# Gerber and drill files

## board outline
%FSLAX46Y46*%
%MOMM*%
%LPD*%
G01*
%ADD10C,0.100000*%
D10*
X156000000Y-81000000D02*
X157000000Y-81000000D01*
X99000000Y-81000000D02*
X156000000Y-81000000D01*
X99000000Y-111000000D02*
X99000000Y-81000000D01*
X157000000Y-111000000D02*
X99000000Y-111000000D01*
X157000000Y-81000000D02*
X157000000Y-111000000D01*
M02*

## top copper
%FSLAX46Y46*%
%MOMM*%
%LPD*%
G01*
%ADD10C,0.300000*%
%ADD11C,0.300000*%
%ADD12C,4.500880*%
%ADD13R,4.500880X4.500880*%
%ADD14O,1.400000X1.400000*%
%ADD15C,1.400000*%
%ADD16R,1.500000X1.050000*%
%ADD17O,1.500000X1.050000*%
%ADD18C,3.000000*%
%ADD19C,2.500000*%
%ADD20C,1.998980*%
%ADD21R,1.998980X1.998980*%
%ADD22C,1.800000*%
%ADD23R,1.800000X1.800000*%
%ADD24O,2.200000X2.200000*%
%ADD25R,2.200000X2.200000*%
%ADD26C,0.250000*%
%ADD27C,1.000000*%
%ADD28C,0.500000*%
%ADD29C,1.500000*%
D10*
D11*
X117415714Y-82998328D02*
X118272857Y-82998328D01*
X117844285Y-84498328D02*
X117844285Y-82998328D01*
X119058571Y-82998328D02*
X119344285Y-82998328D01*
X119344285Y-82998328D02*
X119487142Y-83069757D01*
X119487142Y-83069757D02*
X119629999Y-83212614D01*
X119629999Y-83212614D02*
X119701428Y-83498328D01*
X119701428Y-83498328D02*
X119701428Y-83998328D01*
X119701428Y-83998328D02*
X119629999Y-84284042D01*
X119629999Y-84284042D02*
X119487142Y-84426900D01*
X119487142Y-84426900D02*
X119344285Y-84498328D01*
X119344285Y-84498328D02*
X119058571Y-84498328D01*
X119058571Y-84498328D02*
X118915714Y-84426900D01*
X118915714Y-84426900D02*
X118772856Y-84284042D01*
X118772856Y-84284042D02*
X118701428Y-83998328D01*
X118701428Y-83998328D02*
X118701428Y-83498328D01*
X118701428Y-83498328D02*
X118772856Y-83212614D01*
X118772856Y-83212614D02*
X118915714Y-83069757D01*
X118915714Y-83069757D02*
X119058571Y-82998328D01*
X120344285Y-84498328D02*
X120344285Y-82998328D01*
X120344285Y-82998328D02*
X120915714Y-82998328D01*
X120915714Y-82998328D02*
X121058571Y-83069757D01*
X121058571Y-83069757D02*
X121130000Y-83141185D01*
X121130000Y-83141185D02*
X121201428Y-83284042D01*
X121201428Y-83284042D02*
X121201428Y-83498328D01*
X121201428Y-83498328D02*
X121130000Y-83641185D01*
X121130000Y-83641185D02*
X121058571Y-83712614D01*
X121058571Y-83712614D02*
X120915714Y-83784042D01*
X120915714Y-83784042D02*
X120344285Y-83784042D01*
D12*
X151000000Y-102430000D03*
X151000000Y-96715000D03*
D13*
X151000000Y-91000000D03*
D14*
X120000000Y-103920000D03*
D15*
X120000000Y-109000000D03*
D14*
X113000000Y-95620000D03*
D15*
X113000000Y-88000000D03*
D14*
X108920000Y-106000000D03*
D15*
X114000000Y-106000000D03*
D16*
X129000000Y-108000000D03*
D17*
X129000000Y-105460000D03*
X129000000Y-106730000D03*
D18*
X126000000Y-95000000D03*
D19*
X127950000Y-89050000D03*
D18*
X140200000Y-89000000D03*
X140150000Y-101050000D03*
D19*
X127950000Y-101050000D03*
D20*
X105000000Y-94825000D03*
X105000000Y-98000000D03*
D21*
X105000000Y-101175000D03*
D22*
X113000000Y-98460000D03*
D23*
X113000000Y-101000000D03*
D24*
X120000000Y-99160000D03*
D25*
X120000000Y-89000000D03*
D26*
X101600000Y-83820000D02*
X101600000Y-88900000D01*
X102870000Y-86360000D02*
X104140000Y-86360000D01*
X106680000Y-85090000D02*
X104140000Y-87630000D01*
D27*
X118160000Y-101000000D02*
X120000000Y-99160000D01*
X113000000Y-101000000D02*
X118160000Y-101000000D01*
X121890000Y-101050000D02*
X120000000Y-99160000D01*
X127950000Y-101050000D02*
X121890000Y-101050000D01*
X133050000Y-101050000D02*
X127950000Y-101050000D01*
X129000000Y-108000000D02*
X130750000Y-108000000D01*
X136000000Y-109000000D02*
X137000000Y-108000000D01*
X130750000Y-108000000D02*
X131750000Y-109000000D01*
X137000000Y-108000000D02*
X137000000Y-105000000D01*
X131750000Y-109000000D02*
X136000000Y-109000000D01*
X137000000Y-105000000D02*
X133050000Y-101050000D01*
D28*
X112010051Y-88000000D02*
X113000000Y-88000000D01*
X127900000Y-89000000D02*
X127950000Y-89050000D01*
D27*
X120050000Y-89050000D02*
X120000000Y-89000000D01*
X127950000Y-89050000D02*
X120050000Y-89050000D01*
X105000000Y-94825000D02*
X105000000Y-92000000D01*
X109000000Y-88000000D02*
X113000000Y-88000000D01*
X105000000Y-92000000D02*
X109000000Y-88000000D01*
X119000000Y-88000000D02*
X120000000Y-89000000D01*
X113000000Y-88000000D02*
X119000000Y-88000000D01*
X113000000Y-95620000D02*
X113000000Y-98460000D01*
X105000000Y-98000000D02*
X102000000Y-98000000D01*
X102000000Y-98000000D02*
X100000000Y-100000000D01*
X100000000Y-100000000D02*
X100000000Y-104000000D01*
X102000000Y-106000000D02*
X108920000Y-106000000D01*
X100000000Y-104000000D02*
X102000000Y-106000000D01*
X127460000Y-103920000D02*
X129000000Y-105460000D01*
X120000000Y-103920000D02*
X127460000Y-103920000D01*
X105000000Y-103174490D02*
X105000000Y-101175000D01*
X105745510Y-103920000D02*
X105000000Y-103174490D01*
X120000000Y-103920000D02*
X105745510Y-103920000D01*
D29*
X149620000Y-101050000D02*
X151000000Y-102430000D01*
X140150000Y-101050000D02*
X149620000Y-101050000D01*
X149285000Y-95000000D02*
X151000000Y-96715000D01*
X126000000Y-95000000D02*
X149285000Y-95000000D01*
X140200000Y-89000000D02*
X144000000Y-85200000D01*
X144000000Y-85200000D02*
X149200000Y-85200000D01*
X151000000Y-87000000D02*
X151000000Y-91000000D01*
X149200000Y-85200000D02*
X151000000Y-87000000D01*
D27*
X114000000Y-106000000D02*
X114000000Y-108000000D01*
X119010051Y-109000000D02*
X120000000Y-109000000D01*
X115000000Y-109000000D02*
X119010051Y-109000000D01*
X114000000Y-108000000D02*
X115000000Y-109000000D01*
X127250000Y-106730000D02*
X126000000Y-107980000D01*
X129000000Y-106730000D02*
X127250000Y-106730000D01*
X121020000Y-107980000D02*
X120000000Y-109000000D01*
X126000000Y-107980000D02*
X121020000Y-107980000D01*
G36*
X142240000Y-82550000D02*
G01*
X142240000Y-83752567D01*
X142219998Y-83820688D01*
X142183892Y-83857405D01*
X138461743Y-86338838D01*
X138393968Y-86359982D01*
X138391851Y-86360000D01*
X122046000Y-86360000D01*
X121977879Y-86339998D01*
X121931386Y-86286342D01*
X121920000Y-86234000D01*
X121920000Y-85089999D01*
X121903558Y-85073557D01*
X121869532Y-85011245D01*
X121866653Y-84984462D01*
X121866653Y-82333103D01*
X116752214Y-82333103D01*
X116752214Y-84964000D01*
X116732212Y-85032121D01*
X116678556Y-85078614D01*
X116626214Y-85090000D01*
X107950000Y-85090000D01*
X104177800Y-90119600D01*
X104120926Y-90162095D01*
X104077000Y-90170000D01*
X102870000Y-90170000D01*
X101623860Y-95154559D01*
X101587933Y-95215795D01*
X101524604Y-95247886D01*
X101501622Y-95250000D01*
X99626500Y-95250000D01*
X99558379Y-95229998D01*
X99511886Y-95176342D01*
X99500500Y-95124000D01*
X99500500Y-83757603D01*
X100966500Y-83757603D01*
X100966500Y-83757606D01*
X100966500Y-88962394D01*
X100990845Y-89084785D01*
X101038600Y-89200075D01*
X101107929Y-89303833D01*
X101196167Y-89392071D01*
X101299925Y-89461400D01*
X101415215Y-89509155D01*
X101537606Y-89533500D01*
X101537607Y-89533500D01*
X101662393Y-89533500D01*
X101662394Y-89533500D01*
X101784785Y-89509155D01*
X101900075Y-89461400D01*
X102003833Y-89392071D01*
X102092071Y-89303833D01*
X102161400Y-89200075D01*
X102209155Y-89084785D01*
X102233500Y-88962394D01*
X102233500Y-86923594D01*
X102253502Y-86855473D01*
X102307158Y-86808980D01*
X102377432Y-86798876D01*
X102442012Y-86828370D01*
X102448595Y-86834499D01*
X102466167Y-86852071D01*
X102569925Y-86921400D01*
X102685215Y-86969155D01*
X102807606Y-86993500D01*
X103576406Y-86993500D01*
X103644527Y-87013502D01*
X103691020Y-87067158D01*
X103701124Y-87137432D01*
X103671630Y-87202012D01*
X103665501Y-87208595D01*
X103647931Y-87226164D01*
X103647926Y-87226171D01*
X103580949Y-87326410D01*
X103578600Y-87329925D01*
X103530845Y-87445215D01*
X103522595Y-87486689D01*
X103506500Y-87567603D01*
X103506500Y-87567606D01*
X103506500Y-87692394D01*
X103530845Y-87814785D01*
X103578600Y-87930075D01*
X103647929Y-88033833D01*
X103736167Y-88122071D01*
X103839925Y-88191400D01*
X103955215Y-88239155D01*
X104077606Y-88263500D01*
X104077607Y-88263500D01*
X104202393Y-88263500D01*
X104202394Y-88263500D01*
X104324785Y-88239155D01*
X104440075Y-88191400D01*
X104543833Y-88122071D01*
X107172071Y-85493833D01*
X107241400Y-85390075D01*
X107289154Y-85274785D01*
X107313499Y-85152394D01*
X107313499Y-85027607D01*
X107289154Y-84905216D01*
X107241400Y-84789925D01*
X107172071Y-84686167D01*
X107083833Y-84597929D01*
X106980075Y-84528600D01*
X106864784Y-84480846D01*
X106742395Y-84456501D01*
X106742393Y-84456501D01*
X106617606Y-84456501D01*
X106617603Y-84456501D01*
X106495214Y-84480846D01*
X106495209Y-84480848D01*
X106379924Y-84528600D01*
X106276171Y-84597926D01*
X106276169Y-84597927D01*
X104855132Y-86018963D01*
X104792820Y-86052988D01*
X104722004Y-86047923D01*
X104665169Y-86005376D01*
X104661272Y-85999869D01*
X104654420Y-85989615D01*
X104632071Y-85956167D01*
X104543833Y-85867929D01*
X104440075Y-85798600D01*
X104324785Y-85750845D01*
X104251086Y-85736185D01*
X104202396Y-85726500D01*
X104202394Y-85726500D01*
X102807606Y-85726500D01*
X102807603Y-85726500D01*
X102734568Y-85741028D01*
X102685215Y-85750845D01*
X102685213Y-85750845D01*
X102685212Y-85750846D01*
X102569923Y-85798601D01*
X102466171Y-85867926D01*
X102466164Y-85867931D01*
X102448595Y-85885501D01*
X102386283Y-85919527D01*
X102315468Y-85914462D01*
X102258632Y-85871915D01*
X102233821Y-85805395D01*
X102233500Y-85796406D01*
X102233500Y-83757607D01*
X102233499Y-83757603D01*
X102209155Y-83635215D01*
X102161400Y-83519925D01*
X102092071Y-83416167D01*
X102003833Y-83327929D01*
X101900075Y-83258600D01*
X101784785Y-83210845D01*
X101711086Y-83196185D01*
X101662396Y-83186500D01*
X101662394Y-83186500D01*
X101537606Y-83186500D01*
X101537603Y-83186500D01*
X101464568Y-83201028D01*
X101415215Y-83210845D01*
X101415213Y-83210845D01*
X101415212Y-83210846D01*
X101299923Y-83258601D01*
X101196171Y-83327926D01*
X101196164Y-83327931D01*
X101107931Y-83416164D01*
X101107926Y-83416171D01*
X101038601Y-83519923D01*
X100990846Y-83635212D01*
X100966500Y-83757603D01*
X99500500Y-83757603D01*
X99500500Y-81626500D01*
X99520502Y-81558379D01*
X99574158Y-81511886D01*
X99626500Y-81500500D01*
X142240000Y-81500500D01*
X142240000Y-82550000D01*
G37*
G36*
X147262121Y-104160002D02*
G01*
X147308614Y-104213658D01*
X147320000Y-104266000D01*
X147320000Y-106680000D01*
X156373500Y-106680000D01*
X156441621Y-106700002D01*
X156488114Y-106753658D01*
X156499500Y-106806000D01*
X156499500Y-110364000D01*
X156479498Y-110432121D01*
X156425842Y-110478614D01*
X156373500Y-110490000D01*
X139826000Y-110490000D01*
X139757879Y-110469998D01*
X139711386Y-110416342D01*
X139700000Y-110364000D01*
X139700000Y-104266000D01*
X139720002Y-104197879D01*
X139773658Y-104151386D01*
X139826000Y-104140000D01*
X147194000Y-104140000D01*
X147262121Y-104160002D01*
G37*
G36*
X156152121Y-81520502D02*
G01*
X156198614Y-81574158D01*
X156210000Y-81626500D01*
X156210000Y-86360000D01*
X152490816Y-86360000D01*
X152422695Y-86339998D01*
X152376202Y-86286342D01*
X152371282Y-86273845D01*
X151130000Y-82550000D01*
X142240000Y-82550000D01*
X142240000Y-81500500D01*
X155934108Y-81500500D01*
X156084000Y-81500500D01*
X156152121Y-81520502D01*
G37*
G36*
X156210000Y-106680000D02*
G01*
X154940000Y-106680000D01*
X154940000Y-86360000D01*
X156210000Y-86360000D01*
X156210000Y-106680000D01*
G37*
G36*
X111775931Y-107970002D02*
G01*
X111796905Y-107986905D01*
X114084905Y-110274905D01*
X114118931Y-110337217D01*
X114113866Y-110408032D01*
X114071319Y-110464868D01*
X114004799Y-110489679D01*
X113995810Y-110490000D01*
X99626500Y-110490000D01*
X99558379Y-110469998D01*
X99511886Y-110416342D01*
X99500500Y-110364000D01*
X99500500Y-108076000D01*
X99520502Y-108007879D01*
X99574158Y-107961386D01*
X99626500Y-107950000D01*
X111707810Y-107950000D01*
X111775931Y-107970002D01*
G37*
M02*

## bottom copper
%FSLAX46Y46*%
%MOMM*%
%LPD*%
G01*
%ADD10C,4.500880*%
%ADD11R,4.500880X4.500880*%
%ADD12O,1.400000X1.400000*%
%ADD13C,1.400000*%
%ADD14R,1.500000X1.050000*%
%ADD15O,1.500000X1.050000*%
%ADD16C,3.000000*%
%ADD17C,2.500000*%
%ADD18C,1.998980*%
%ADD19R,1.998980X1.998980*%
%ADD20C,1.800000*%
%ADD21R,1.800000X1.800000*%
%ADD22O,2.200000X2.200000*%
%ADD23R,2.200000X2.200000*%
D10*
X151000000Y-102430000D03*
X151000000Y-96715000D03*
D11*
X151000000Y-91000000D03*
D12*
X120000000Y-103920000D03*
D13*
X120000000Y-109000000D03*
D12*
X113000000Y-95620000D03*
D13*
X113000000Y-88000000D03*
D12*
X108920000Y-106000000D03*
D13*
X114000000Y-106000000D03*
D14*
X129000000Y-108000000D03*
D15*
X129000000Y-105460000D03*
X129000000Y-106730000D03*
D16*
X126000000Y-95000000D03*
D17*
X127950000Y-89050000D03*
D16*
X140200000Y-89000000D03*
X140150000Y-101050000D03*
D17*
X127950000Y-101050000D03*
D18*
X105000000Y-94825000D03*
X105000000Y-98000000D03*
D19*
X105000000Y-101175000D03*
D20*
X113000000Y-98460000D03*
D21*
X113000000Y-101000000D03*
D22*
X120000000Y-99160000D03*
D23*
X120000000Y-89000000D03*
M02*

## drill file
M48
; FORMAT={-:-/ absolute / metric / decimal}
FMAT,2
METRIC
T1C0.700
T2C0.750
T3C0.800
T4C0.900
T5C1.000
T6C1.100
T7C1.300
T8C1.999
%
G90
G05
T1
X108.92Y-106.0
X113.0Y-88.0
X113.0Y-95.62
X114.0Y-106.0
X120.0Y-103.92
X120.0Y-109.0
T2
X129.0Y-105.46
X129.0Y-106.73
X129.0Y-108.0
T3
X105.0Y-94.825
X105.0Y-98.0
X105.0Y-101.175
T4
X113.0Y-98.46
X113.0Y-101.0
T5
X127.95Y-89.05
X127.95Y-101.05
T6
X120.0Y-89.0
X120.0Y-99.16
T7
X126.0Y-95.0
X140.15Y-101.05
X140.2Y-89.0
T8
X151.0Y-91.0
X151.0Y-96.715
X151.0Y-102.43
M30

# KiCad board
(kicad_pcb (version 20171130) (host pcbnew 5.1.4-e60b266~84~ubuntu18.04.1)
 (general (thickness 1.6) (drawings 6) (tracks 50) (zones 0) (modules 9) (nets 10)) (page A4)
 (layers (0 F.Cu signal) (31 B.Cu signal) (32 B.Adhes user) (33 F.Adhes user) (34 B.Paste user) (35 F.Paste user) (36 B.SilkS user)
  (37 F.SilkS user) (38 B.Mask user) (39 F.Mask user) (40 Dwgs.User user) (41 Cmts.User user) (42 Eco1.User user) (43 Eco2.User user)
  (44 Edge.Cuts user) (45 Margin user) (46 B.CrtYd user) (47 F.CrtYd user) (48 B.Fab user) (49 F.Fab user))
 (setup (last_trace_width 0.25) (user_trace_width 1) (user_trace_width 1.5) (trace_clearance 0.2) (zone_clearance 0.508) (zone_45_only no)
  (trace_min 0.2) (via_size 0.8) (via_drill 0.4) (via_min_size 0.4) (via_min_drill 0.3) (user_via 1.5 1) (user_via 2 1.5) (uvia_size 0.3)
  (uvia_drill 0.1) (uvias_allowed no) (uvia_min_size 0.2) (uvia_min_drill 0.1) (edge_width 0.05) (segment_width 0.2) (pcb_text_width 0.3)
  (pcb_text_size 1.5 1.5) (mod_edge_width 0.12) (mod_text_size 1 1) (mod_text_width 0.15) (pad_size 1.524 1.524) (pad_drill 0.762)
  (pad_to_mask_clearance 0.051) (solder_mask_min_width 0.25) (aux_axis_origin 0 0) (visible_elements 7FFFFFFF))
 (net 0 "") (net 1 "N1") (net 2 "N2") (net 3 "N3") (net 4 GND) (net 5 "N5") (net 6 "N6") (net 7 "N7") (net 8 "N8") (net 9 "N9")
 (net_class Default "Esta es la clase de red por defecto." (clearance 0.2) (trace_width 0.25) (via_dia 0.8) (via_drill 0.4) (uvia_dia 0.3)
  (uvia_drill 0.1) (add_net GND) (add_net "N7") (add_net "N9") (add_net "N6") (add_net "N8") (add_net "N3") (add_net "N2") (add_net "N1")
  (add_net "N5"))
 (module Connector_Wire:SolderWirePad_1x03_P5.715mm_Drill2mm (layer F.Cu) (at 151 91 270)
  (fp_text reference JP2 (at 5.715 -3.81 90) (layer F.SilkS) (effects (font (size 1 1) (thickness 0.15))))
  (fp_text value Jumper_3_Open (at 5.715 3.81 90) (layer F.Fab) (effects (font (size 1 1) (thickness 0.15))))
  (pad 3 thru_hole circle (at 11.43 0 270) (size 4.50088 4.50088) (drill 1.99898) (layers *.Cu *.Mask) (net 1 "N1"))
  (pad 2 thru_hole circle (at 5.715 0 270) (size 4.50088 4.50088) (drill 1.99898) (layers *.Cu *.Mask) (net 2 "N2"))
  (pad 1 thru_hole rect (at 0 0 270) (size 4.50088 4.50088) (drill 1.99898) (layers *.Cu *.Mask) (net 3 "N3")))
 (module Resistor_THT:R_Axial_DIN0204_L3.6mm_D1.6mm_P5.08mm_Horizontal (layer F.Cu) (at 120 109 90)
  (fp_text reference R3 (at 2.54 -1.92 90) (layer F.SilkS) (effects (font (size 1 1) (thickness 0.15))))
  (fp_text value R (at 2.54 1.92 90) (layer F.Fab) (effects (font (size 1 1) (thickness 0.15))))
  (pad 2 thru_hole oval (at 5.08 0 90) (size 1.4 1.4) (drill 0.7) (layers *.Cu *.Mask) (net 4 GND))
  (pad 1 thru_hole circle (at 0 0 90) (size 1.4 1.4) (drill 0.7) (layers *.Cu *.Mask) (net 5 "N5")))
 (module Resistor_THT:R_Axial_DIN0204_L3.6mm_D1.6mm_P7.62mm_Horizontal (layer F.Cu) (at 113 88 270)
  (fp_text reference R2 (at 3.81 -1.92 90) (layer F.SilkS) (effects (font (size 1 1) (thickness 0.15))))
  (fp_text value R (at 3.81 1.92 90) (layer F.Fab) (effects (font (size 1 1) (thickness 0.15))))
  (pad 2 thru_hole oval (at 7.62 0 270) (size 1.4 1.4) (drill 0.7) (layers *.Cu *.Mask) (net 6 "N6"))
  (pad 1 thru_hole circle (at 0 0 270) (size 1.4 1.4) (drill 0.7) (layers *.Cu *.Mask) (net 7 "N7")))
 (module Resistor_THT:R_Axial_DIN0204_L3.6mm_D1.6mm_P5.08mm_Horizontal (layer F.Cu) (at 114 106 180)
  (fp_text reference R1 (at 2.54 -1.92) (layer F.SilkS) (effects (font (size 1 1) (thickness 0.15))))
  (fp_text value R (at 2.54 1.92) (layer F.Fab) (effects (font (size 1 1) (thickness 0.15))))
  (pad 2 thru_hole oval (at 5.08 0 180) (size 1.4 1.4) (drill 0.7) (layers *.Cu *.Mask) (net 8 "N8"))
  (pad 1 thru_hole circle (at 0 0 180) (size 1.4 1.4) (drill 0.7) (layers *.Cu *.Mask) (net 5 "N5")))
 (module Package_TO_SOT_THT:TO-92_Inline (layer F.Cu) (at 129 108 90)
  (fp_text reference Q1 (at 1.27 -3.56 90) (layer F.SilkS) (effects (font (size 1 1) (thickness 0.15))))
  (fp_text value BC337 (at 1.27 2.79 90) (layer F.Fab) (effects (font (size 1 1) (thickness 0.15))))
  (pad 1 thru_hole rect (at 0 0 90) (size 1.05 1.5) (drill 0.75) (layers *.Cu *.Mask) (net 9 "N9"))
  (pad 3 thru_hole oval (at 2.54 0 90) (size 1.05 1.5) (drill 0.75) (layers *.Cu *.Mask) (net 4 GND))
  (pad 2 thru_hole oval (at 1.27 0 90) (size 1.05 1.5) (drill 0.75) (layers *.Cu *.Mask) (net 5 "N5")))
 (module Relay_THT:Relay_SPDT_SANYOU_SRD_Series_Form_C (layer F.Cu) (at 126 95)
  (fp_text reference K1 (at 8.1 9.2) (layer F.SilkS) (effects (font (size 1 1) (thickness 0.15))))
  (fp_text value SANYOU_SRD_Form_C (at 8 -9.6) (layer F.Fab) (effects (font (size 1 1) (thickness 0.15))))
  (pad 1 thru_hole circle (at 0 0 90) (size 3 3) (drill 1.3) (layers *.Cu *.Mask) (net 2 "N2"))
  (pad 5 thru_hole circle (at 1.95 -5.95 90) (size 2.5 2.5) (drill 1) (layers *.Cu *.Mask) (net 7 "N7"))
  (pad 4 thru_hole circle (at 14.2 -6 90) (size 3 3) (drill 1.3) (layers *.Cu *.Mask) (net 3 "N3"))
  (pad 3 thru_hole circle (at 14.15 6.05 90) (size 3 3) (drill 1.3) (layers *.Cu *.Mask) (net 1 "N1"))
  (pad 2 thru_hole circle (at 1.95 6.05 90) (size 2.5 2.5) (drill 1) (layers *.Cu *.Mask) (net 9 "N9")))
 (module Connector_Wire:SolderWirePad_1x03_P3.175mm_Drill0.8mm (layer F.Cu) (at 105 101.175 90)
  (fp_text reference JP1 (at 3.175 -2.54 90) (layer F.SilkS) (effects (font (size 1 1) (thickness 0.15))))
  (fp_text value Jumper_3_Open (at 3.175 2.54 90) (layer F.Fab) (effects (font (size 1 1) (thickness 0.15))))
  (pad 3 thru_hole circle (at 6.35 0 90) (size 1.99898 1.99898) (drill 0.8001) (layers *.Cu *.Mask) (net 7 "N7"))
  (pad 2 thru_hole circle (at 3.175 0 90) (size 1.99898 1.99898) (drill 0.8001) (layers *.Cu *.Mask) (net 8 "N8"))
  (pad 1 thru_hole rect (at 0 0 90) (size 1.99898 1.99898) (drill 0.8001) (layers *.Cu *.Mask) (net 4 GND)))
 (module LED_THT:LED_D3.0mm (layer F.Cu) (at 113 101 90)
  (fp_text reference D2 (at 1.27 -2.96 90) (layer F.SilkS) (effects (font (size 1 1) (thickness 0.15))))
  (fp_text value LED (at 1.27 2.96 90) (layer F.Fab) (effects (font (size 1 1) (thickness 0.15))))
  (pad 2 thru_hole circle (at 2.54 0 90) (size 1.8 1.8) (drill 0.9) (layers *.Cu *.Mask) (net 6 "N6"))
  (pad 1 thru_hole rect (at 0 0 90) (size 1.8 1.8) (drill 0.9) (layers *.Cu *.Mask) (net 9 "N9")))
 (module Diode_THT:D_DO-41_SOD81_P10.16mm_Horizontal (layer F.Cu) (at 120 89 270)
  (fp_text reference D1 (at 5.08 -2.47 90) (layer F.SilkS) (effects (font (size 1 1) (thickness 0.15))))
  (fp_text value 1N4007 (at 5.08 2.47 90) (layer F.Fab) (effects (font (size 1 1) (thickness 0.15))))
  (pad 2 thru_hole oval (at 10.16 0 270) (size 2.2 2.2) (drill 1.1) (layers *.Cu *.Mask) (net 9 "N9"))
  (pad 1 thru_hole rect (at 0 0 270) (size 2.2 2.2) (drill 1.1) (layers *.Cu *.Mask) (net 7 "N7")))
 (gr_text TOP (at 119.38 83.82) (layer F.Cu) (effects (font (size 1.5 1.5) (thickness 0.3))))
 (gr_line (start 156 81) (end 157 81) (layer Edge.Cuts) (width 0.1))
 (gr_line (start 99 81) (end 156 81) (layer Edge.Cuts) (width 0.1))
 (gr_line (start 99 111) (end 99 81) (layer Edge.Cuts) (width 0.1))
 (gr_line (start 157 111) (end 99 111) (layer Edge.Cuts) (width 0.1))
 (gr_line (start 157 81) (end 157 111) (layer Edge.Cuts) (width 0.1))
 (segment (start 101.6 83.82) (end 101.6 88.9) (width 0.25) (layer F.Cu) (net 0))
 (segment (start 102.87 86.36) (end 104.14 86.36) (width 0.25) (layer F.Cu) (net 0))
 (segment (start 106.68 85.09) (end 104.14 87.63) (width 0.25) (layer F.Cu) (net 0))
 (segment (start 118.16 101) (end 120 99.16) (width 1) (layer F.Cu) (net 9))
 (segment (start 113 101) (end 118.16 101) (width 1) (layer F.Cu) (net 9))
 (segment (start 121.89 101.05) (end 120 99.16) (width 1) (layer F.Cu) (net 9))
 (segment (start 127.95 101.05) (end 121.89 101.05) (width 1) (layer F.Cu) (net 9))
 (segment (start 133.05 101.05) (end 127.95 101.05) (width 1) (layer F.Cu) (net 9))
 (segment (start 129 108) (end 130.75 108) (width 1) (layer F.Cu) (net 9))
 (segment (start 136 109) (end 137 108) (width 1) (layer F.Cu) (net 9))
 (segment (start 130.75 108) (end 131.75 109) (width 1) (layer F.Cu) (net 9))
 (segment (start 137 108) (end 137 105) (width 1) (layer F.Cu) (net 9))
 (segment (start 131.75 109) (end 136 109) (width 1) (layer F.Cu) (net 9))
 (segment (start 137 105) (end 133.05 101.05) (width 1) (layer F.Cu) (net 9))
 (segment (start 112.010051 88) (end 113 88) (width 0.5) (layer F.Cu) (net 7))
 (segment (start 127.9 89) (end 127.95 89.05) (width 0.5) (layer F.Cu) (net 7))
 (segment (start 120.05 89.05) (end 120 89) (width 1) (layer F.Cu) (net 7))
 (segment (start 127.95 89.05) (end 120.05 89.05) (width 1) (layer F.Cu) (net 7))
 (segment (start 105 94.825) (end 105 92) (width 1) (layer F.Cu) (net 7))
 (segment (start 109 88) (end 113 88) (width 1) (layer F.Cu) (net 7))
 (segment (start 105 92) (end 109 88) (width 1) (layer F.Cu) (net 7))
 (segment (start 119 88) (end 120 89) (width 1) (layer F.Cu) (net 7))
 (segment (start 113 88) (end 119 88) (width 1) (layer F.Cu) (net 7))
 (segment (start 113 95.62) (end 113 98.46) (width 1) (layer F.Cu) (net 6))
 (segment (start 105 98) (end 102 98) (width 1) (layer F.Cu) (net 8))
 (segment (start 102 98) (end 100 100) (width 1) (layer F.Cu) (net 8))
 (segment (start 100 100) (end 100 104) (width 1) (layer F.Cu) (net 8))
 (segment (start 102 106) (end 108.92 106) (width 1) (layer F.Cu) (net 8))
 (segment (start 100 104) (end 102 106) (width 1) (layer F.Cu) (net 8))
 (segment (start 127.46 103.92) (end 129 105.46) (width 1) (layer F.Cu) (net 4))
 (segment (start 120 103.92) (end 127.46 103.92) (width 1) (layer F.Cu) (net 4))
 (segment (start 105 103.17449) (end 105 101.175) (width 1) (layer F.Cu) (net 4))
 (segment (start 105.74551 103.92) (end 105 103.17449) (width 1) (layer F.Cu) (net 4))
 (segment (start 120 103.92) (end 105.74551 103.92) (width 1) (layer F.Cu) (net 4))
 (segment (start 149.62 101.05) (end 151 102.43) (width 1.5) (layer F.Cu) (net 1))
 (segment (start 140.15 101.05) (end 149.62 101.05) (width 1.5) (layer F.Cu) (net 1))
 (segment (start 149.285 95) (end 151 96.715) (width 1.5) (layer F.Cu) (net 2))
 (segment (start 126 95) (end 149.285 95) (width 1.5) (layer F.Cu) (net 2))
 (segment (start 140.2 89) (end 144 85.2) (width 1.5) (layer F.Cu) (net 3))
 (segment (start 144 85.2) (end 149.2 85.2) (width 1.5) (layer F.Cu) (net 3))
 (segment (start 151 87) (end 151 91) (width 1.5) (layer F.Cu) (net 3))
 (segment (start 149.2 85.2) (end 151 87) (width 1.5) (layer F.Cu) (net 3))
 (segment (start 114 106) (end 114 108) (width 1) (layer F.Cu) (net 5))
 (segment (start 119.010051 109) (end 120 109) (width 1) (layer F.Cu) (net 5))
 (segment (start 115 109) (end 119.010051 109) (width 1) (layer F.Cu) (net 5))
 (segment (start 114 108) (end 115 109) (width 1) (layer F.Cu) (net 5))
 (segment (start 127.25 106.73) (end 126 107.98) (width 1) (layer F.Cu) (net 5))
 (segment (start 129 106.73) (end 127.25 106.73) (width 1) (layer F.Cu) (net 5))
 (segment (start 121.02 107.98) (end 120 109) (width 1) (layer F.Cu) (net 5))
 (segment (start 126 107.98) (end 121.02 107.98) (width 1) (layer F.Cu) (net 5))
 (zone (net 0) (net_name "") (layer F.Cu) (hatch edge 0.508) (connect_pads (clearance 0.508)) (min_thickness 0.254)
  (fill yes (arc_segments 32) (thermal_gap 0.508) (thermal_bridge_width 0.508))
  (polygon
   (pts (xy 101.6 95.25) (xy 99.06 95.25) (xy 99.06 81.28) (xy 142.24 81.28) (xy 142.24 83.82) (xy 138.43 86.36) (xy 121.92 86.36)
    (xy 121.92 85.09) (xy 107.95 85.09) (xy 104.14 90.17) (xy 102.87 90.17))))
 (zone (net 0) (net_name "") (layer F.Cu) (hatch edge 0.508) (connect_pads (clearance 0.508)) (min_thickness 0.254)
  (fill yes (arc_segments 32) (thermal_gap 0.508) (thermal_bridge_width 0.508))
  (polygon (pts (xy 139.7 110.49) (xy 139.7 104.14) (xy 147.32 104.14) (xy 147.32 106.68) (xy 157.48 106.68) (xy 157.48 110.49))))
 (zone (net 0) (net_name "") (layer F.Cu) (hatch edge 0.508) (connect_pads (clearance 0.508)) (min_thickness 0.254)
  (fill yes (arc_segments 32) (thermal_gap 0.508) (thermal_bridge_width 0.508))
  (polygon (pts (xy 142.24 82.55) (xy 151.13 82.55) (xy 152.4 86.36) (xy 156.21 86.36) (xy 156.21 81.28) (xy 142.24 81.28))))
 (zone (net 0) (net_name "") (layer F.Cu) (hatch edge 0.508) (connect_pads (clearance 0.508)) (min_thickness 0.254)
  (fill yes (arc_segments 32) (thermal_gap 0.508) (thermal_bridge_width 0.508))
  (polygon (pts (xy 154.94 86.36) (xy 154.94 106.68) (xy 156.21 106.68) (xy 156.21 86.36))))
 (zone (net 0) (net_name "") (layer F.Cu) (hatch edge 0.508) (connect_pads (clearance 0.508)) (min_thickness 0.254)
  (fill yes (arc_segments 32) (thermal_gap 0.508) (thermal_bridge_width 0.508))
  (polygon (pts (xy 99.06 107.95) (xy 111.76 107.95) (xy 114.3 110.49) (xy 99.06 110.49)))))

